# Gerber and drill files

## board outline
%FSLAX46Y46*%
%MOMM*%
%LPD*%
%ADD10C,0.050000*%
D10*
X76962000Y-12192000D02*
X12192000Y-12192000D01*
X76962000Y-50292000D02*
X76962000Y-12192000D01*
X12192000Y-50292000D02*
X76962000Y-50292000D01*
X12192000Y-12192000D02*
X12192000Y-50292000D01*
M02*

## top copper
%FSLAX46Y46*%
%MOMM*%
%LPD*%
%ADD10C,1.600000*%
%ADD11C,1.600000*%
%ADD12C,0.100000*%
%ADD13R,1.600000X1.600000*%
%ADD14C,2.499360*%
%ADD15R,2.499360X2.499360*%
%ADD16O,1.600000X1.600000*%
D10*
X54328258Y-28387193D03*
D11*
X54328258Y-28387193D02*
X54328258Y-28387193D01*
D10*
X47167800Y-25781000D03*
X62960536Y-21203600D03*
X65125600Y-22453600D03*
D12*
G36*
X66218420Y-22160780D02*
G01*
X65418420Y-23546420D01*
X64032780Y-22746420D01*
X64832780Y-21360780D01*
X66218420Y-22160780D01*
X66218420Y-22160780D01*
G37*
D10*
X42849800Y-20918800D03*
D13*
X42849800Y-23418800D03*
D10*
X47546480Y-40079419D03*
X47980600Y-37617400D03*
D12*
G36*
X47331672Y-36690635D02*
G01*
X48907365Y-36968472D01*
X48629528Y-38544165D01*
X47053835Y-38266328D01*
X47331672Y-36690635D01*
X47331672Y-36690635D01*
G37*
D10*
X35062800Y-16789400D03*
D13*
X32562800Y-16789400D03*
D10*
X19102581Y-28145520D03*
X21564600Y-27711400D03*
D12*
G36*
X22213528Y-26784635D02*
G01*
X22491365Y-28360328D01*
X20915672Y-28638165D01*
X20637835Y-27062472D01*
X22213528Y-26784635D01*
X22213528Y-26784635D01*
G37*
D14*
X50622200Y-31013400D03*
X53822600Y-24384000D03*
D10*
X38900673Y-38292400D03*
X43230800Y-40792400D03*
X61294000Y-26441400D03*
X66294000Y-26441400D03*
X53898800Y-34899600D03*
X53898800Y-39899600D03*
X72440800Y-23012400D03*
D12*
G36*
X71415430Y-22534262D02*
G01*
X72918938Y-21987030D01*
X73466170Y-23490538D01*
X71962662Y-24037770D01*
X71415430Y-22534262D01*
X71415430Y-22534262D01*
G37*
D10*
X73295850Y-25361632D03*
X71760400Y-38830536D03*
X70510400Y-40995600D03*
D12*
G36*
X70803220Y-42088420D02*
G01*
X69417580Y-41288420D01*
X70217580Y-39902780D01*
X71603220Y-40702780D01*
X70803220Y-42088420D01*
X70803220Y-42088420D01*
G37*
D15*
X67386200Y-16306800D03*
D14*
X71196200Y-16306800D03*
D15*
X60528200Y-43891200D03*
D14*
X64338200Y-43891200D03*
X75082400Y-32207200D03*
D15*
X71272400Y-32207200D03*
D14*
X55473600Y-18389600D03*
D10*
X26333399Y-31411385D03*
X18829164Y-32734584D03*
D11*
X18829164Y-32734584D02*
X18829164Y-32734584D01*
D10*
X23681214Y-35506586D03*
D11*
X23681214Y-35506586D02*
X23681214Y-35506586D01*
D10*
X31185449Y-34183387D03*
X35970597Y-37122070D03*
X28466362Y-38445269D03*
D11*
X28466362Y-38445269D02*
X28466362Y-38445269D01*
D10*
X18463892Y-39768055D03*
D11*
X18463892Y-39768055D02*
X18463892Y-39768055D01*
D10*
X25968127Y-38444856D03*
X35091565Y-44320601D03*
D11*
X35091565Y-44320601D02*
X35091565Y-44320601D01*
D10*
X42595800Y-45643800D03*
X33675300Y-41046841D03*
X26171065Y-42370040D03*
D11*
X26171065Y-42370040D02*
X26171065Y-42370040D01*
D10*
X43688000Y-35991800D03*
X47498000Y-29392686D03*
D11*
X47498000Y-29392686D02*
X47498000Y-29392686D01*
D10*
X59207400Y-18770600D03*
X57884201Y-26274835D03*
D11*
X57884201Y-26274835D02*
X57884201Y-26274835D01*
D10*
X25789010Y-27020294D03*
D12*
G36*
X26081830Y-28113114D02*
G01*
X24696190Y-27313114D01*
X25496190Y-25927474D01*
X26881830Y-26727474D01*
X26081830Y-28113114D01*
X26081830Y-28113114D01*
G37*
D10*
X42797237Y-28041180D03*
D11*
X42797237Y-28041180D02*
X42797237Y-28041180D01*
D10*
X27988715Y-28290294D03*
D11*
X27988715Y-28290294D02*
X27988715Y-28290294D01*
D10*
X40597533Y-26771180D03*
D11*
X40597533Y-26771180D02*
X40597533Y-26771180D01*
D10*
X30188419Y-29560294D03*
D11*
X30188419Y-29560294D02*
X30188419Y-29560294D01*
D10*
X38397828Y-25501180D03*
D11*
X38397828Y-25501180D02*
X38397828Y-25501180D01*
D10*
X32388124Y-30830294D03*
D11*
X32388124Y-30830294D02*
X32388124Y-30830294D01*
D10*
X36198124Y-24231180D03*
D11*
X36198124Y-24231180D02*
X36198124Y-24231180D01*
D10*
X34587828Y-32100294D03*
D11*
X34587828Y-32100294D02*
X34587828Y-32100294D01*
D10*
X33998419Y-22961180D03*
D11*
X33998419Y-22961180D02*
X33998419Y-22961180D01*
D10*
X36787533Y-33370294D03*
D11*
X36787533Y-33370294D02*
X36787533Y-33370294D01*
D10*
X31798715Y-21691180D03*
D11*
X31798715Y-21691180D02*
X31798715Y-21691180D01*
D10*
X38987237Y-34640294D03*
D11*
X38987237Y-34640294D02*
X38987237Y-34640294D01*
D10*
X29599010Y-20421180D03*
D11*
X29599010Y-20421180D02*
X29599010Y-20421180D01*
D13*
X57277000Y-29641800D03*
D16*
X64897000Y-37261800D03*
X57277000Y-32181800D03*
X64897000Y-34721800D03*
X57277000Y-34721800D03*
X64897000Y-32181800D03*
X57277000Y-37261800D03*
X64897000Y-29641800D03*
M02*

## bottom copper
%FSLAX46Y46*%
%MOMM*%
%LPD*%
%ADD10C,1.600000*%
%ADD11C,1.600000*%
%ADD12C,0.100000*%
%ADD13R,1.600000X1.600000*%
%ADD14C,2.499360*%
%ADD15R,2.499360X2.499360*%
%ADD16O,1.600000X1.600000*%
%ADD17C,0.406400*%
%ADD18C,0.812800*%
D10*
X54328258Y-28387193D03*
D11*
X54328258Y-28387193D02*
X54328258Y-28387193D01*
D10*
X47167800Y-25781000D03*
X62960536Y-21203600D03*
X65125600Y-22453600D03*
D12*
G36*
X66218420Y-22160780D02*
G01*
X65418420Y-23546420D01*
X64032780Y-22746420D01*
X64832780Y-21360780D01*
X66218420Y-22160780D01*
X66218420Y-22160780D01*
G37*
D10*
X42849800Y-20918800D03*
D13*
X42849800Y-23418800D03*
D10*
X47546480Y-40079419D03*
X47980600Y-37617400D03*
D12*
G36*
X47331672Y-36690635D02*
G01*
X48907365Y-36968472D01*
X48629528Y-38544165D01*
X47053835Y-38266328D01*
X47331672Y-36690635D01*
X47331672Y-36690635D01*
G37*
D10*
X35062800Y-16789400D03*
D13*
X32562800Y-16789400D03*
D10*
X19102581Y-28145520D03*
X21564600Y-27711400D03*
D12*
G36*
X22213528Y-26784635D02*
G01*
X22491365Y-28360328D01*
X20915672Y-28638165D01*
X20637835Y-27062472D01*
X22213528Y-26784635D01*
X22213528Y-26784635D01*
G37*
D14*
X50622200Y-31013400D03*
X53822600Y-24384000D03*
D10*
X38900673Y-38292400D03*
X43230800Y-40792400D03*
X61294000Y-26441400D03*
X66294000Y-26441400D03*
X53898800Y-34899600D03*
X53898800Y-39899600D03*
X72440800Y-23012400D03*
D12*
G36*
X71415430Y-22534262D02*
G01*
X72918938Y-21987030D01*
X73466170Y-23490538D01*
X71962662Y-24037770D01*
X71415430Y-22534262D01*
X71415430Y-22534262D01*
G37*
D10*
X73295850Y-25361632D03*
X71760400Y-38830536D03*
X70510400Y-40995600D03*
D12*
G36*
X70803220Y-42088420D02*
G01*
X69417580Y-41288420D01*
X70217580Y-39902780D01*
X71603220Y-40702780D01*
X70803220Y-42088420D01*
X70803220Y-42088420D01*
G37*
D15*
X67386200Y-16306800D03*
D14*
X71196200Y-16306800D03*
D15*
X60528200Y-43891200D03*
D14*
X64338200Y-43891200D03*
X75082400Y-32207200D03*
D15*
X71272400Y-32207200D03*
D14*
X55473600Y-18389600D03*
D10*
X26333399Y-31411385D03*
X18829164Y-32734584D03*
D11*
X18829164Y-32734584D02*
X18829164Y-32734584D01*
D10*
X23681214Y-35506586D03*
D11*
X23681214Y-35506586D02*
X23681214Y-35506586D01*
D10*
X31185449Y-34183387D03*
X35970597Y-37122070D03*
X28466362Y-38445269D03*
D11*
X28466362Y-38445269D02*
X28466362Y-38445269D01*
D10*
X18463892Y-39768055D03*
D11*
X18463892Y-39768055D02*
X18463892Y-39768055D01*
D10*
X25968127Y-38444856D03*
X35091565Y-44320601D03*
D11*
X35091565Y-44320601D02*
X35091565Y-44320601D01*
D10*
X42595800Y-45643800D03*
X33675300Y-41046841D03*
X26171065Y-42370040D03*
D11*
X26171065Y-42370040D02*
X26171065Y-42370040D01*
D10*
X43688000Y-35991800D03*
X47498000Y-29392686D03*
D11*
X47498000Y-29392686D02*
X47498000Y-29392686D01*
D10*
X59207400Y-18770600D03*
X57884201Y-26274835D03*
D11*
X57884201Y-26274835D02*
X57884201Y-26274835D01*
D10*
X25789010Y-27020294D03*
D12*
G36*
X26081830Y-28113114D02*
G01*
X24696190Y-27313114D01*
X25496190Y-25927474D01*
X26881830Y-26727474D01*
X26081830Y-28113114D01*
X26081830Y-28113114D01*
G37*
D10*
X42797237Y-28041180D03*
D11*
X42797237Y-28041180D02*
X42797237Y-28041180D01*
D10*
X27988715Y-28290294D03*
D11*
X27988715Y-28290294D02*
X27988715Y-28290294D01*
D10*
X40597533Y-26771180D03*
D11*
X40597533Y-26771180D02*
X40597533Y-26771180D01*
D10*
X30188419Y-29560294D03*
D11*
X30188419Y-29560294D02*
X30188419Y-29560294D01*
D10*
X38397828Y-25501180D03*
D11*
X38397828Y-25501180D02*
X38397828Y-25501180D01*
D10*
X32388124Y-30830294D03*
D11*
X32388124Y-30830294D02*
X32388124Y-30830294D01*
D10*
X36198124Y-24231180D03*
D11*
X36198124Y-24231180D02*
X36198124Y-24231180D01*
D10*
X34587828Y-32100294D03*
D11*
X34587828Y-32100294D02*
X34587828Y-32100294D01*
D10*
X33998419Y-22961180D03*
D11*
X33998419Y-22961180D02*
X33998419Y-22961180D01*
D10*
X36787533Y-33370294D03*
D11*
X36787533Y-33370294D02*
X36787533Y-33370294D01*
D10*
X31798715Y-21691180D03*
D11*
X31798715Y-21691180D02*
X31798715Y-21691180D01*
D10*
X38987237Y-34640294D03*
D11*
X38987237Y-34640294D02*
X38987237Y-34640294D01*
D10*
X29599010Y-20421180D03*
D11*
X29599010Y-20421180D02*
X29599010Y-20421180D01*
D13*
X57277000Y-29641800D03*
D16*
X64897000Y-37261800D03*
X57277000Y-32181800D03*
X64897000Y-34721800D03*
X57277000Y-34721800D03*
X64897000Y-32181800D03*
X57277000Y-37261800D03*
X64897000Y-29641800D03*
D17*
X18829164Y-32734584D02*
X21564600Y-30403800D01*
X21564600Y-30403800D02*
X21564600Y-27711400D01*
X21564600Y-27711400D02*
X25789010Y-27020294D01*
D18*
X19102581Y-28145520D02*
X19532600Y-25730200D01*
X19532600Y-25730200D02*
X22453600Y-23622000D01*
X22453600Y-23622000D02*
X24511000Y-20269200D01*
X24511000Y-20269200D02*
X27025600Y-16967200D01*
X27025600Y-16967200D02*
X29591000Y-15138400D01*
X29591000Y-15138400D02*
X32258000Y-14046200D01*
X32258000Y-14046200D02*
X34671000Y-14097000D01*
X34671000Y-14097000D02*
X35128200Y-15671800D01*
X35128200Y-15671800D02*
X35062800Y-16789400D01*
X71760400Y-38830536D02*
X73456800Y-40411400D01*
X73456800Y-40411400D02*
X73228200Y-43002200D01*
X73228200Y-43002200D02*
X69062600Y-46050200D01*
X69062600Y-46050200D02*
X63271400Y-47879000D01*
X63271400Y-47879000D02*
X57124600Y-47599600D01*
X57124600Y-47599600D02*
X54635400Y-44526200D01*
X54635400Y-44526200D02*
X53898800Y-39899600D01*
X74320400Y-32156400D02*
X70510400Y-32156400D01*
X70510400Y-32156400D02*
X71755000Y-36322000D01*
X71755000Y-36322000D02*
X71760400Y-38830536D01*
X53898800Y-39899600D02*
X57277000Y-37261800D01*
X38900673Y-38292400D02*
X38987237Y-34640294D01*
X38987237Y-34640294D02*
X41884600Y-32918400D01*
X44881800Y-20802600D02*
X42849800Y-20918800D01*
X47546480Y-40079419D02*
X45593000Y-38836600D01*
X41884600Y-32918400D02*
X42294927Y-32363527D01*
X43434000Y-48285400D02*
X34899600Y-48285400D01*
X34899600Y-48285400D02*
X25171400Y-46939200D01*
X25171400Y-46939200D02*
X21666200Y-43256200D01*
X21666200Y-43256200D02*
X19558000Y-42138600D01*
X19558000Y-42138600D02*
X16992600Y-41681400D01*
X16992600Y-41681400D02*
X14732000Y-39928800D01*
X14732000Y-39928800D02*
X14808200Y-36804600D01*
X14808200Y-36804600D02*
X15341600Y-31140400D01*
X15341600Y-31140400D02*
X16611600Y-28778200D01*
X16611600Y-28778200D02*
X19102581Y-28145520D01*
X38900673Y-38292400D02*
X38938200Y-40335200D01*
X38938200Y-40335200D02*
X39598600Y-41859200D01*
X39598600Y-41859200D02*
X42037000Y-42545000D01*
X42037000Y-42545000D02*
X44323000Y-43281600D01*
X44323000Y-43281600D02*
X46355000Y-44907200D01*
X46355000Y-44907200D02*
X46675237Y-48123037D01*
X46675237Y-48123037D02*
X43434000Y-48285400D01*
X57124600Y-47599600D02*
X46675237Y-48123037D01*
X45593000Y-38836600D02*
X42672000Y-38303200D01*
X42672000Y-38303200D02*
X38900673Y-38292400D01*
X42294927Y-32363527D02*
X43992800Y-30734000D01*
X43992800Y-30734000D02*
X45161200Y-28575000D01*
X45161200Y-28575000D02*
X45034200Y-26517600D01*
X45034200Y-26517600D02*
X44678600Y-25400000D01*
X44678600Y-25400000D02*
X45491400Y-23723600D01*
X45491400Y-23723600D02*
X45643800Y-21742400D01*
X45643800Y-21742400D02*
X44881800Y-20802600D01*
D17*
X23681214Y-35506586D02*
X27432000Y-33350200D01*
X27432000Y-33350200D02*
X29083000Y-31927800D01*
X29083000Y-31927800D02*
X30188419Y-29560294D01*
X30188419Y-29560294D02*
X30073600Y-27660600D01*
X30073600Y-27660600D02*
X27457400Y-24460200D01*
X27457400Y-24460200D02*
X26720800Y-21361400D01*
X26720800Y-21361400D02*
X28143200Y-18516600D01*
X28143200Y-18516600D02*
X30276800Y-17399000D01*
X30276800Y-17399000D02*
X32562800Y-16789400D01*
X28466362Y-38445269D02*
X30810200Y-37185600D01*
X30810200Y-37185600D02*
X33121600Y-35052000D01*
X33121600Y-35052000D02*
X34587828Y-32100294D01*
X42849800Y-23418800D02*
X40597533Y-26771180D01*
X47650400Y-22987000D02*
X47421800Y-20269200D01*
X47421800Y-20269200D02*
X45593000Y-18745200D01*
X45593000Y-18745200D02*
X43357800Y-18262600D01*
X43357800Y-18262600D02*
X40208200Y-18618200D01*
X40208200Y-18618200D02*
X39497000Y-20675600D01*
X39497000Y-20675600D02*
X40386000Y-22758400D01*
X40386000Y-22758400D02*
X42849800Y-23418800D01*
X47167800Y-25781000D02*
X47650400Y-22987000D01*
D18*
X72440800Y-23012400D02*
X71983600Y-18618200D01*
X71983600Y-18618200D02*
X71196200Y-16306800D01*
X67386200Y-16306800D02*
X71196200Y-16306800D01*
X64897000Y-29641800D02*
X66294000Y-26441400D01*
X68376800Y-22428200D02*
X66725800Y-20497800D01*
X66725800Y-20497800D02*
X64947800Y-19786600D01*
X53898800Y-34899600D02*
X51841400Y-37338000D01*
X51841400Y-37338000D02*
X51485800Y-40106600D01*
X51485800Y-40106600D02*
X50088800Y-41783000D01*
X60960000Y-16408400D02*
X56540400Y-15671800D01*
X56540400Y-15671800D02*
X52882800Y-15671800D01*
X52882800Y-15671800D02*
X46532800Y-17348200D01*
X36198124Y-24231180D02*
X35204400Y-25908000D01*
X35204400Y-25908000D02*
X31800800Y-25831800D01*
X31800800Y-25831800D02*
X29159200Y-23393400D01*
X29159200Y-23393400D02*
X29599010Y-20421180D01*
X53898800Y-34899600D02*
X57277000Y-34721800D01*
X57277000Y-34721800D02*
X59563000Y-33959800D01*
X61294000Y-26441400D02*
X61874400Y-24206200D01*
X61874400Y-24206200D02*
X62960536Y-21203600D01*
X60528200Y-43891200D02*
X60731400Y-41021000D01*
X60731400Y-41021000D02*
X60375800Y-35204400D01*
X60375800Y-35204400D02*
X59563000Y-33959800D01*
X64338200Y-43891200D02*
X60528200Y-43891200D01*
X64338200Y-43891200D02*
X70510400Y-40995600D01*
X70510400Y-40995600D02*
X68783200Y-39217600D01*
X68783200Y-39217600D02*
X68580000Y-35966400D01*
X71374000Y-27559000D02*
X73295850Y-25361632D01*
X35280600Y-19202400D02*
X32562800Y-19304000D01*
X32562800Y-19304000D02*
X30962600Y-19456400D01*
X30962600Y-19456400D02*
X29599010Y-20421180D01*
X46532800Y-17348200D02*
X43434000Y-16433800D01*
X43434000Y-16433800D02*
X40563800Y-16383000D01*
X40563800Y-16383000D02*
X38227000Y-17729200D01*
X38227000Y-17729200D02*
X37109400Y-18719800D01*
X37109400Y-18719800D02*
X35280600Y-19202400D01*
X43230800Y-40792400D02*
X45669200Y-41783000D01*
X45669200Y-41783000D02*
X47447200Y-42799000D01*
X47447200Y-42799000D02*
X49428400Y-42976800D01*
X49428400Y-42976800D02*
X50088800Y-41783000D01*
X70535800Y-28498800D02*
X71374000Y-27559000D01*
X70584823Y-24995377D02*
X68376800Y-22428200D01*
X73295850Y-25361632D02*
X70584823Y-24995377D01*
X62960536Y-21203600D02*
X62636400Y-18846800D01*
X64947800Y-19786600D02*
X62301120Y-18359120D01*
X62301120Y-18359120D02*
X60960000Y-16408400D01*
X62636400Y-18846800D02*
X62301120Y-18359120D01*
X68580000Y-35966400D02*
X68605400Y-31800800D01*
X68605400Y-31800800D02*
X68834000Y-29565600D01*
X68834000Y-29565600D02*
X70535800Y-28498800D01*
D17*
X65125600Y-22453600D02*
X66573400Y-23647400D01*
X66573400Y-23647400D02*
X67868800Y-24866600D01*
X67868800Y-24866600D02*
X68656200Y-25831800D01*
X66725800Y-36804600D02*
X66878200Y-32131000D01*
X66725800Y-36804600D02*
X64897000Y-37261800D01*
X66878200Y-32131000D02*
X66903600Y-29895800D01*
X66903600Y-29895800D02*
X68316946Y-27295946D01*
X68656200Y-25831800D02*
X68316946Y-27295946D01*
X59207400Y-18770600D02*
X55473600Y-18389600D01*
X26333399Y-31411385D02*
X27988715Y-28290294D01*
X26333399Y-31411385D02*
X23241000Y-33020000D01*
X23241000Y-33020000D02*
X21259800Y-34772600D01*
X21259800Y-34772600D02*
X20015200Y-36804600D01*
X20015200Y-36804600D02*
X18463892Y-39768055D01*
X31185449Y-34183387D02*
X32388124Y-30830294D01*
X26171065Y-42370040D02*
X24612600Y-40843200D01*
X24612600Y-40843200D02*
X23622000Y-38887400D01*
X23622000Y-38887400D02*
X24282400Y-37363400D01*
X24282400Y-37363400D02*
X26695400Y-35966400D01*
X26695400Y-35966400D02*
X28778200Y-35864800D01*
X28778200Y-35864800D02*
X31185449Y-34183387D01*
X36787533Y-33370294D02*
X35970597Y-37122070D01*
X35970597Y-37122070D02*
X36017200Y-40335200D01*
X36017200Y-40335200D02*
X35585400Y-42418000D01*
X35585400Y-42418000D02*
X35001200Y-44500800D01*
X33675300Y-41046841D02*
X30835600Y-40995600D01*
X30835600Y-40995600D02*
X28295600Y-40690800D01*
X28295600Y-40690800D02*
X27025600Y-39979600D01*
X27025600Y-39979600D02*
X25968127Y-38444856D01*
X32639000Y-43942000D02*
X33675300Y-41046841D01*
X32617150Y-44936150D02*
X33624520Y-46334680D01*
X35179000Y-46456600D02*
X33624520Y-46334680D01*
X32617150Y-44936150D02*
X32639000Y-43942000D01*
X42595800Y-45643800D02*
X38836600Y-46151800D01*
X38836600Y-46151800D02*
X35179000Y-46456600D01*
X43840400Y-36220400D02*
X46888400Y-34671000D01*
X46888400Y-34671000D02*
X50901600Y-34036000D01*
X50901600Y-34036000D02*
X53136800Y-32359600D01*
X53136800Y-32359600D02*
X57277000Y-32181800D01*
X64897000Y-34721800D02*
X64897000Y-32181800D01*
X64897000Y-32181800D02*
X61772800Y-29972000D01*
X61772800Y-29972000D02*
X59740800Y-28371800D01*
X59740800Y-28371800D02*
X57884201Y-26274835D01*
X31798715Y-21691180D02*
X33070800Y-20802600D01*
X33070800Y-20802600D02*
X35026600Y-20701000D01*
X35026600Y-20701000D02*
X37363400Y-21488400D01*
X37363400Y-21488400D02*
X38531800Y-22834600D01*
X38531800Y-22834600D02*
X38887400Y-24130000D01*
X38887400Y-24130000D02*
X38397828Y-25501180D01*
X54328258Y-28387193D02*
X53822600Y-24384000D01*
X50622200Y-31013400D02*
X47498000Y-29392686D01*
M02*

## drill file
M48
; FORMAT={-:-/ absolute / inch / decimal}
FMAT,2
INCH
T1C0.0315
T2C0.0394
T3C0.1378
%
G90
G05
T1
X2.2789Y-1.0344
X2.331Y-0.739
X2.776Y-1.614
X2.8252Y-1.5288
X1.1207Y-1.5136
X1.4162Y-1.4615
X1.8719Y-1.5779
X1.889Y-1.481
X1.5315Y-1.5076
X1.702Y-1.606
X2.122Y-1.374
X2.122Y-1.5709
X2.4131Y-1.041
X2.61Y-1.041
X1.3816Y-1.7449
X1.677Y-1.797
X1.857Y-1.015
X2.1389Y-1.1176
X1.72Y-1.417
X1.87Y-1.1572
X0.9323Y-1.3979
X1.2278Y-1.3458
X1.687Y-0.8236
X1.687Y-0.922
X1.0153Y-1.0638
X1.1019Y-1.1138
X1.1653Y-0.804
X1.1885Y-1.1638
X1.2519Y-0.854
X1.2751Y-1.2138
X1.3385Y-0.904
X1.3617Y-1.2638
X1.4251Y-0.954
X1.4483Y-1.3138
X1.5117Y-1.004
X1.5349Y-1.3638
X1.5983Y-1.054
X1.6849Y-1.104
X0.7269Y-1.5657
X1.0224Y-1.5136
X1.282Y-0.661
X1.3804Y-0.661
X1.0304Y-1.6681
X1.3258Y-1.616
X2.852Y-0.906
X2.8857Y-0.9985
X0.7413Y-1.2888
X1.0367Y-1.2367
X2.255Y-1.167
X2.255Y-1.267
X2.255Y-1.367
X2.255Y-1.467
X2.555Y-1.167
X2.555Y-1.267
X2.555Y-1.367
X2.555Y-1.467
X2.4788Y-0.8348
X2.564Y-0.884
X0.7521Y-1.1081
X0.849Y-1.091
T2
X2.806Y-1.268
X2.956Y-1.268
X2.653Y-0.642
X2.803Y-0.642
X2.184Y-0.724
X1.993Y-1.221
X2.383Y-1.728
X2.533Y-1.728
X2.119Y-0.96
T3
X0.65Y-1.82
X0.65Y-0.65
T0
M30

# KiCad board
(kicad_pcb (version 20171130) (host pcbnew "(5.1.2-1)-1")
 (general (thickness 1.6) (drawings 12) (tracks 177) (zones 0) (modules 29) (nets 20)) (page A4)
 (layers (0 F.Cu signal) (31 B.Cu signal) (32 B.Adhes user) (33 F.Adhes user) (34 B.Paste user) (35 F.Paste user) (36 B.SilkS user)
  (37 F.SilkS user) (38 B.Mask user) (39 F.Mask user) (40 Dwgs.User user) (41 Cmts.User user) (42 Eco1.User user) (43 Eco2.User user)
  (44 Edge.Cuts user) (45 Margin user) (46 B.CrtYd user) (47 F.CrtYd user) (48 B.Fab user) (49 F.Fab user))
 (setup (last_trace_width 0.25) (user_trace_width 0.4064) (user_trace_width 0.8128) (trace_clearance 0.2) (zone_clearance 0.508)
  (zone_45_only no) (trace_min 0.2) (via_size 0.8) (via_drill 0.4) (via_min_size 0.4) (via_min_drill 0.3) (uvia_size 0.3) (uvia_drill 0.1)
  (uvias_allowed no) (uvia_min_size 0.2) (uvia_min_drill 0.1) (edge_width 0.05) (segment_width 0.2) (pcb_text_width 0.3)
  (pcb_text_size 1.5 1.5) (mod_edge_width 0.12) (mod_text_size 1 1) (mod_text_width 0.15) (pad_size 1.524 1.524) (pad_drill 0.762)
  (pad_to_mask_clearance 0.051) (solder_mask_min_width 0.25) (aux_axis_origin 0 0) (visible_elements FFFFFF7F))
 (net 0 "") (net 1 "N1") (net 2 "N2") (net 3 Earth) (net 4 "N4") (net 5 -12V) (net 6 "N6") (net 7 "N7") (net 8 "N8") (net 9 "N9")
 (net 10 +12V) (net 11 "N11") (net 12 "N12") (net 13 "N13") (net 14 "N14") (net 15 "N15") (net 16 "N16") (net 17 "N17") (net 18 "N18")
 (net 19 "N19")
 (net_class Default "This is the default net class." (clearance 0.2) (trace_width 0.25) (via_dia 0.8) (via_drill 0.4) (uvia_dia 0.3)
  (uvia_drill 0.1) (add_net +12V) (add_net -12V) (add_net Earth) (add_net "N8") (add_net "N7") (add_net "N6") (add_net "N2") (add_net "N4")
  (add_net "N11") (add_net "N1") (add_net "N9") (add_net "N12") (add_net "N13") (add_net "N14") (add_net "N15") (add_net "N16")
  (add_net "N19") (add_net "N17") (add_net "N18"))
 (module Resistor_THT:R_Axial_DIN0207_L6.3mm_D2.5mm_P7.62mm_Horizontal (layer F.Cu) (at 47.1678 25.781 340)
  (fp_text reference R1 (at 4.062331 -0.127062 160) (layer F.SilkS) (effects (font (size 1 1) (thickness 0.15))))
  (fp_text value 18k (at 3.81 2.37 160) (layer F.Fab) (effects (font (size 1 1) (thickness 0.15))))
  (pad 2 thru_hole oval (at 7.62 0 340) (size 1.6 1.6) (drill 0.8) (layers *.Cu *.Mask) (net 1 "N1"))
  (pad 1 thru_hole circle (at 0 0 340) (size 1.6 1.6) (drill 0.8) (layers *.Cu *.Mask) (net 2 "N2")))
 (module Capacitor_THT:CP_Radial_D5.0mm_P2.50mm (layer F.Cu) (at 65.1256 22.4536 150)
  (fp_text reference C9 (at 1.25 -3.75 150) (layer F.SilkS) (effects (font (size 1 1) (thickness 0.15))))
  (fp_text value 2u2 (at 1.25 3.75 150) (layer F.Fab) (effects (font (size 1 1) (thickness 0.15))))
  (pad 2 thru_hole circle (at 2.5 0 150) (size 1.6 1.6) (drill 0.8) (layers *.Cu *.Mask) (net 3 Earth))
  (pad 1 thru_hole rect (at 0 0 150) (size 1.6 1.6) (drill 0.8) (layers *.Cu *.Mask) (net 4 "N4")))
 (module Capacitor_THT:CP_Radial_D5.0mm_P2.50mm (layer F.Cu) (at 42.8498 23.4188 90)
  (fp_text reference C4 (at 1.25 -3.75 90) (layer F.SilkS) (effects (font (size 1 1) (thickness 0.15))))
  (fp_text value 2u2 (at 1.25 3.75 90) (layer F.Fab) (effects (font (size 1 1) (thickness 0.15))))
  (pad 2 thru_hole circle (at 2.5 0 90) (size 1.6 1.6) (drill 0.8) (layers *.Cu *.Mask) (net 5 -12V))
  (pad 1 thru_hole rect (at 0 0 90) (size 1.6 1.6) (drill 0.8) (layers *.Cu *.Mask) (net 2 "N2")))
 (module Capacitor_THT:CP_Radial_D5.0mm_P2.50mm (layer F.Cu) (at 47.9806 37.6174 260)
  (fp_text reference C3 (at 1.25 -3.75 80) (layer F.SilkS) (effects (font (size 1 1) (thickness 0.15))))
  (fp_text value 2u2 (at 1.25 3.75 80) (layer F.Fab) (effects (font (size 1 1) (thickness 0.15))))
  (pad 2 thru_hole circle (at 2.5 0 260) (size 1.6 1.6) (drill 0.8) (layers *.Cu *.Mask) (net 5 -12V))
  (pad 1 thru_hole rect (at 0 0 260) (size 1.6 1.6) (drill 0.8) (layers *.Cu *.Mask) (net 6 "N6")))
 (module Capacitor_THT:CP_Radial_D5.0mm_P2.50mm (layer F.Cu) (at 32.5628 16.7894)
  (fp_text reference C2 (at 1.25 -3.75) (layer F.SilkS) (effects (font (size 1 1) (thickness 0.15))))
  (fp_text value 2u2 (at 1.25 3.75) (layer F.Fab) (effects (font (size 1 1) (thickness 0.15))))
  (pad 2 thru_hole circle (at 2.5 0) (size 1.6 1.6) (drill 0.8) (layers *.Cu *.Mask) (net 5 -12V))
  (pad 1 thru_hole rect (at 0 0) (size 1.6 1.6) (drill 0.8) (layers *.Cu *.Mask) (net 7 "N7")))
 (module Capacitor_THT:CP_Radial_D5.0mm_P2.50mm (layer F.Cu) (at 21.5646 27.7114 190)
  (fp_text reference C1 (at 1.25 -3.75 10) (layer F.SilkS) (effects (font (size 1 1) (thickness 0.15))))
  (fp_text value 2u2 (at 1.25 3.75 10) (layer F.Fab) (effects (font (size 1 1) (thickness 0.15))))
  (pad 2 thru_hole circle (at 2.5 0 190) (size 1.6 1.6) (drill 0.8) (layers *.Cu *.Mask) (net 5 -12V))
  (pad 1 thru_hole rect (at 0 0 190) (size 1.6 1.6) (drill 0.8) (layers *.Cu *.Mask) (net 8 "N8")))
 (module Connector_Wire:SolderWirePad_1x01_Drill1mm (layer F.Cu) (at 50.6222 31.0134 340)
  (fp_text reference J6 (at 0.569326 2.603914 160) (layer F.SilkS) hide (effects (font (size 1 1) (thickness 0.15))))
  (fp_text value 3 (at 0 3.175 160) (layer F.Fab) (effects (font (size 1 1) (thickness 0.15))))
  (pad 1 thru_hole circle (at 0 0 340) (size 2.49936 2.49936) (drill 1.00076) (layers *.Cu *.Mask) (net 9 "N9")))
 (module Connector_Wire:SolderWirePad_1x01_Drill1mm (layer F.Cu) (at 53.8226 24.384 340)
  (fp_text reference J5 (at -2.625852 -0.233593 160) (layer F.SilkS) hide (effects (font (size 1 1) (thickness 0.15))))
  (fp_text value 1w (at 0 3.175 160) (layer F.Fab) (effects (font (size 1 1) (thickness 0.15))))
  (pad 1 thru_hole circle (at 0 0 340) (size 2.49936 2.49936) (drill 1.00076) (layers *.Cu *.Mask) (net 1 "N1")))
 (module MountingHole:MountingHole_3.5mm (layer F.Cu) (at 16.51 46.228)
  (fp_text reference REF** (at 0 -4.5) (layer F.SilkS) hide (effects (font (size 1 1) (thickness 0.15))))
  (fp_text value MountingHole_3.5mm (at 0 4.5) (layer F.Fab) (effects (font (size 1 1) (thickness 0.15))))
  (pad 1 np_thru_hole circle (at 0 0) (size 3.5 3.5) (drill 3.5) (layers *.Cu *.Mask)))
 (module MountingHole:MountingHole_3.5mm (layer F.Cu) (at 16.51 16.51)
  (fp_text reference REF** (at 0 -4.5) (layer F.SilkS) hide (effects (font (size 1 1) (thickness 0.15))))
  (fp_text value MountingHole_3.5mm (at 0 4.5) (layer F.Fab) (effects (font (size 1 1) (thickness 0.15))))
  (pad 1 np_thru_hole circle (at 0 0) (size 3.5 3.5) (drill 3.5) (layers *.Cu *.Mask)))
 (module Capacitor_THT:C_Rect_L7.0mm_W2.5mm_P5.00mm (layer F.Cu) (at 43.2308 40.7924 150)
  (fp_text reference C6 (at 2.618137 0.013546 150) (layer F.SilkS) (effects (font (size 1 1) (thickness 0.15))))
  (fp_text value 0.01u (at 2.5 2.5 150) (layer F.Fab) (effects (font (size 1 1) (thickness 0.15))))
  (pad 2 thru_hole circle (at 5 0 150) (size 1.6 1.6) (drill 0.8) (layers *.Cu *.Mask) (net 5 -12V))
  (pad 1 thru_hole circle (at 0 0 150) (size 1.6 1.6) (drill 0.8) (layers *.Cu *.Mask) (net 3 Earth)))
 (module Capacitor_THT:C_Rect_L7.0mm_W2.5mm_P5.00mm (layer F.Cu) (at 66.294 26.4414 180)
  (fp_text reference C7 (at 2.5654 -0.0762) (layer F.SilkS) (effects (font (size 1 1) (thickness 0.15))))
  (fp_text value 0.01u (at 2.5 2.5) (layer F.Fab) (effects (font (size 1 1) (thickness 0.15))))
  (pad 2 thru_hole circle (at 5 0 180) (size 1.6 1.6) (drill 0.8) (layers *.Cu *.Mask) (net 3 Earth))
  (pad 1 thru_hole circle (at 0 0 180) (size 1.6 1.6) (drill 0.8) (layers *.Cu *.Mask) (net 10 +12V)))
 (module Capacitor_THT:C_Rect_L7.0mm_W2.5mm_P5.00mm (layer F.Cu) (at 53.8988 34.8996 270)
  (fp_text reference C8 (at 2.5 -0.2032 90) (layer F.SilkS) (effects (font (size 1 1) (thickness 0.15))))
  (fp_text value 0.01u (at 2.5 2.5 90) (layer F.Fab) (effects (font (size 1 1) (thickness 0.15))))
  (pad 1 thru_hole circle (at 0 0 270) (size 1.6 1.6) (drill 0.8) (layers *.Cu *.Mask) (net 3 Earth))
  (pad 2 thru_hole circle (at 5 0 270) (size 1.6 1.6) (drill 0.8) (layers *.Cu *.Mask) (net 5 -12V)))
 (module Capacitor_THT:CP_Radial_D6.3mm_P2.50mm (layer F.Cu) (at 72.4408 23.0124 290)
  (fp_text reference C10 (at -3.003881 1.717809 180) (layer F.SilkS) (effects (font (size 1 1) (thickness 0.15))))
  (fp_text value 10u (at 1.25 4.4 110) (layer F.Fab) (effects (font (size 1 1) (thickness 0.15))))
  (pad 1 thru_hole rect (at 0 0 290) (size 1.6 1.6) (drill 0.8) (layers *.Cu *.Mask) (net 10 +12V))
  (pad 2 thru_hole circle (at 2.5 0 290) (size 1.6 1.6) (drill 0.8) (layers *.Cu *.Mask) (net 3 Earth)))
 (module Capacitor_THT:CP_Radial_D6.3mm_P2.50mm (layer F.Cu) (at 70.5104 40.9956 60)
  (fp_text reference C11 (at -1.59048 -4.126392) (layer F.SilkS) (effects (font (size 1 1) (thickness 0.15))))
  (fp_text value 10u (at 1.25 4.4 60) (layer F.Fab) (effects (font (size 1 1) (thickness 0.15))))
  (pad 2 thru_hole circle (at 2.5 0 60) (size 1.6 1.6) (drill 0.8) (layers *.Cu *.Mask) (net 5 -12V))
  (pad 1 thru_hole rect (at 0 0 60) (size 1.6 1.6) (drill 0.8) (layers *.Cu *.Mask) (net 3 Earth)))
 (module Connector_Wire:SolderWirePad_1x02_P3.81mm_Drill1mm (layer F.Cu) (at 67.3862 16.3068)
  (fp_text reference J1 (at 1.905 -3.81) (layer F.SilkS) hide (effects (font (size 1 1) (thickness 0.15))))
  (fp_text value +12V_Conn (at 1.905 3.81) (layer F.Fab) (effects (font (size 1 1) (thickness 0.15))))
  (pad 1 thru_hole rect (at 0 0) (size 2.49936 2.49936) (drill 1.00076) (layers *.Cu *.Mask) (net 10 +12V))
  (pad 2 thru_hole circle (at 3.81 0) (size 2.49936 2.49936) (drill 1.00076) (layers *.Cu *.Mask) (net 10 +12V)))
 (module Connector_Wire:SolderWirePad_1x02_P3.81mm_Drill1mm (layer F.Cu) (at 60.5282 43.8912)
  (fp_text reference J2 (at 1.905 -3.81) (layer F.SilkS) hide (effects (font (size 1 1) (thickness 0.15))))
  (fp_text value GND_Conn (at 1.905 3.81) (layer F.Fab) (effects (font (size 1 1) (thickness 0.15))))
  (pad 1 thru_hole rect (at 0 0) (size 2.49936 2.49936) (drill 1.00076) (layers *.Cu *.Mask) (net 3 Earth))
  (pad 2 thru_hole circle (at 3.81 0) (size 2.49936 2.49936) (drill 1.00076) (layers *.Cu *.Mask) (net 3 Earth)))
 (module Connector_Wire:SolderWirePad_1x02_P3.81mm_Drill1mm (layer F.Cu) (at 71.2724 32.2072)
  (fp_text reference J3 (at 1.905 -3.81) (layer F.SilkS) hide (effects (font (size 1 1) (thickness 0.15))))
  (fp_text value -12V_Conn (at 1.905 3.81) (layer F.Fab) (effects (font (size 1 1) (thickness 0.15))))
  (pad 2 thru_hole circle (at 3.81 0) (size 2.49936 2.49936) (drill 1.00076) (layers *.Cu *.Mask) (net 5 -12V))
  (pad 1 thru_hole rect (at 0 0) (size 2.49936 2.49936) (drill 1.00076) (layers *.Cu *.Mask) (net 5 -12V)))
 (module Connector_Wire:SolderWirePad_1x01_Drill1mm (layer F.Cu) (at 55.4736 18.3896 350)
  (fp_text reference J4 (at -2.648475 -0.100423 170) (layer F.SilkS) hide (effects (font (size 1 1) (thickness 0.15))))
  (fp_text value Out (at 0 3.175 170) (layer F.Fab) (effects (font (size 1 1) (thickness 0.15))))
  (pad 1 thru_hole circle (at 0 0 350) (size 2.49936 2.49936) (drill 1.00076) (layers *.Cu *.Mask) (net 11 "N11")))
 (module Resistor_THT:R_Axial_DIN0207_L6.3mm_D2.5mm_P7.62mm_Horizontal (layer F.Cu) (at 26.333399 31.411385 190)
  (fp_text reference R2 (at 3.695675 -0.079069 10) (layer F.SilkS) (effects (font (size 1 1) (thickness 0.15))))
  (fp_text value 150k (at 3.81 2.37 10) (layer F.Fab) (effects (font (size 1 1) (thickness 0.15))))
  (pad 1 thru_hole circle (at 0 0 190) (size 1.6 1.6) (drill 0.8) (layers *.Cu *.Mask) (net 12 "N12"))
  (pad 2 thru_hole oval (at 7.62 0 190) (size 1.6 1.6) (drill 0.8) (layers *.Cu *.Mask) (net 8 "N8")))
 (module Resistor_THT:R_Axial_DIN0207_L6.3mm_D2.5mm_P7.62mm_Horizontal (layer F.Cu) (at 31.185449 34.183387 190)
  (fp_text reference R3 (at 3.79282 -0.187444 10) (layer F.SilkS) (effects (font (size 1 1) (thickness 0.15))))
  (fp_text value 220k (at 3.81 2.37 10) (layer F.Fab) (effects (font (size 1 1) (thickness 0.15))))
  (pad 2 thru_hole oval (at 7.62 0 190) (size 1.6 1.6) (drill 0.8) (layers *.Cu *.Mask) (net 7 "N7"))
  (pad 1 thru_hole circle (at 0 0 190) (size 1.6 1.6) (drill 0.8) (layers *.Cu *.Mask) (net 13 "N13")))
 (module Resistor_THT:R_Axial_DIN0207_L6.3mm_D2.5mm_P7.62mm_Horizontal (layer F.Cu) (at 35.970597 37.12207 190)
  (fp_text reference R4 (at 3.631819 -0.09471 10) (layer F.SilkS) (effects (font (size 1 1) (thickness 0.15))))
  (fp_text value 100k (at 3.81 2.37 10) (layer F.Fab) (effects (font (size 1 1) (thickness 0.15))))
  (pad 1 thru_hole circle (at 0 0 190) (size 1.6 1.6) (drill 0.8) (layers *.Cu *.Mask) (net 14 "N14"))
  (pad 2 thru_hole oval (at 7.62 0 190) (size 1.6 1.6) (drill 0.8) (layers *.Cu *.Mask) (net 6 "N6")))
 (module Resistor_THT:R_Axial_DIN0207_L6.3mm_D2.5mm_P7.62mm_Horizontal (layer F.Cu) (at 25.968127 38.444856 190)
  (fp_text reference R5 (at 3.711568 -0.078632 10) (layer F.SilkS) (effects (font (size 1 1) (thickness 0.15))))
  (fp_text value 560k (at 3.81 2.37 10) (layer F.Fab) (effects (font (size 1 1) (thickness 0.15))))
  (pad 2 thru_hole oval (at 7.62 0 190) (size 1.6 1.6) (drill 0.8) (layers *.Cu *.Mask) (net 12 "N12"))
  (pad 1 thru_hole circle (at 0 0 190) (size 1.6 1.6) (drill 0.8) (layers *.Cu *.Mask) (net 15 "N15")))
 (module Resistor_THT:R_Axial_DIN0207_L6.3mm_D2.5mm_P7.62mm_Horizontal (layer F.Cu) (at 42.5958 45.6438 170)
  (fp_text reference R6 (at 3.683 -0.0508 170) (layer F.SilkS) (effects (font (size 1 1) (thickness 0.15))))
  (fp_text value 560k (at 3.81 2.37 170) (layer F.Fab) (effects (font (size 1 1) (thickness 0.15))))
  (pad 2 thru_hole oval (at 7.62 0 170) (size 1.6 1.6) (drill 0.8) (layers *.Cu *.Mask) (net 14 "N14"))
  (pad 1 thru_hole circle (at 0 0 170) (size 1.6 1.6) (drill 0.8) (layers *.Cu *.Mask) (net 15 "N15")))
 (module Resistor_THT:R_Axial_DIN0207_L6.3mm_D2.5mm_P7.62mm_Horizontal (layer F.Cu) (at 33.6753 41.046841 190)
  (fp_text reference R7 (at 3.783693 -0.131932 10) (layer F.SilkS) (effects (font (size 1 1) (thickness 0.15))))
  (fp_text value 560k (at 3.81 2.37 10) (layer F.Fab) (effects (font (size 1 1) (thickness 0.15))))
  (pad 1 thru_hole circle (at 0 0 190) (size 1.6 1.6) (drill 0.8) (layers *.Cu *.Mask) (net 15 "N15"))
  (pad 2 thru_hole oval (at 7.62 0 190) (size 1.6 1.6) (drill 0.8) (layers *.Cu *.Mask) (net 13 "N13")))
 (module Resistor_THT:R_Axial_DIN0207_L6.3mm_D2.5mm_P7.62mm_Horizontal (layer F.Cu) (at 43.688 35.9918 60)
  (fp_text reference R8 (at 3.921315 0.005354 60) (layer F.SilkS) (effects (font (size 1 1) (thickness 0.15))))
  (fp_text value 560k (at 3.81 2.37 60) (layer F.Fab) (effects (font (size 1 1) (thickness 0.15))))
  (pad 1 thru_hole circle (at 0 0 60) (size 1.6 1.6) (drill 0.8) (layers *.Cu *.Mask) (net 15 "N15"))
  (pad 2 thru_hole oval (at 7.62 0 60) (size 1.6 1.6) (drill 0.8) (layers *.Cu *.Mask) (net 9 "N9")))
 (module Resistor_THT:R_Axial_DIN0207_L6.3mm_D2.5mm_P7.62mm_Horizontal (layer F.Cu) (at 59.2074 18.7706 260)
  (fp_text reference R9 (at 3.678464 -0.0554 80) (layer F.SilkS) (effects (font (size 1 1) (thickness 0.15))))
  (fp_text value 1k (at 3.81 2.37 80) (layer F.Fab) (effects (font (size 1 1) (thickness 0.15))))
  (pad 1 thru_hole circle (at 0 0 260) (size 1.6 1.6) (drill 0.8) (layers *.Cu *.Mask) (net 11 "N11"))
  (pad 2 thru_hole oval (at 7.62 0 260) (size 1.6 1.6) (drill 0.8) (layers *.Cu *.Mask) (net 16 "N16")))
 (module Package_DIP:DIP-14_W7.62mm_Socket (layer F.Cu) (at 25.78901 27.020294 60)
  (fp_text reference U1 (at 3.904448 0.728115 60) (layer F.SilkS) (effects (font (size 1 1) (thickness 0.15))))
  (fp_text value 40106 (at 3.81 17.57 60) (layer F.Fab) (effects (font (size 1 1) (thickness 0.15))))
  (pad 1 thru_hole rect (at 0 0 60) (size 1.6 1.6) (drill 0.8) (layers *.Cu *.Mask) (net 8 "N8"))
  (pad 8 thru_hole oval (at 7.62 15.24 60) (size 1.6 1.6) (drill 0.8) (layers *.Cu *.Mask) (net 9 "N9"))
  (pad 2 thru_hole oval (at 0 2.54 60) (size 1.6 1.6) (drill 0.8) (layers *.Cu *.Mask) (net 12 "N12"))
  (pad 9 thru_hole oval (at 7.62 12.7 60) (size 1.6 1.6) (drill 0.8) (layers *.Cu *.Mask) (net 2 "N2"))
  (pad 3 thru_hole oval (at 0 5.08 60) (size 1.6 1.6) (drill 0.8) (layers *.Cu *.Mask) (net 7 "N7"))
  (pad 10 thru_hole oval (at 7.62 10.16 60) (size 1.6 1.6) (drill 0.8) (layers *.Cu *.Mask) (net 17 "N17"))
  (pad 4 thru_hole oval (at 0 7.62 60) (size 1.6 1.6) (drill 0.8) (layers *.Cu *.Mask) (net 13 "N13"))
  (pad 11 thru_hole oval (at 7.62 7.62 60) (size 1.6 1.6) (drill 0.8) (layers *.Cu *.Mask) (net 3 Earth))
  (pad 5 thru_hole oval (at 0 10.16 60) (size 1.6 1.6) (drill 0.8) (layers *.Cu *.Mask) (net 6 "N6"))
  (pad 12 thru_hole oval (at 7.62 5.08 60) (size 1.6 1.6) (drill 0.8) (layers *.Cu *.Mask) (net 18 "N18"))
  (pad 6 thru_hole oval (at 0 12.7 60) (size 1.6 1.6) (drill 0.8) (layers *.Cu *.Mask) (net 14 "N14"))
  (pad 13 thru_hole oval (at 7.62 2.54 60) (size 1.6 1.6) (drill 0.8) (layers *.Cu *.Mask) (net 17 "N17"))
  (pad 7 thru_hole oval (at 0 15.24 60) (size 1.6 1.6) (drill 0.8) (layers *.Cu *.Mask) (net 5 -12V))
  (pad 14 thru_hole oval (at 7.62 0 60) (size 1.6 1.6) (drill 0.8) (layers *.Cu *.Mask) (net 3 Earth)))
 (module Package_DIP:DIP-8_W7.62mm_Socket (layer F.Cu) (at 57.277 29.6418)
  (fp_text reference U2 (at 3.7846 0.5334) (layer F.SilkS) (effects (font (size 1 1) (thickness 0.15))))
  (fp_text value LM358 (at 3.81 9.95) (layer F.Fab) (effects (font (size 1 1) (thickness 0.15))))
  (pad 1 thru_hole rect (at 0 0) (size 1.6 1.6) (drill 0.8) (layers *.Cu *.Mask) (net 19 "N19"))
  (pad 5 thru_hole oval (at 7.62 7.62) (size 1.6 1.6) (drill 0.8) (layers *.Cu *.Mask) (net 4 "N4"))
  (pad 2 thru_hole oval (at 0 2.54) (size 1.6 1.6) (drill 0.8) (layers *.Cu *.Mask) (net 15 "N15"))
  (pad 6 thru_hole oval (at 7.62 5.08) (size 1.6 1.6) (drill 0.8) (layers *.Cu *.Mask) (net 16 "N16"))
  (pad 3 thru_hole oval (at 0 5.08) (size 1.6 1.6) (drill 0.8) (layers *.Cu *.Mask) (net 3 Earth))
  (pad 7 thru_hole oval (at 7.62 2.54) (size 1.6 1.6) (drill 0.8) (layers *.Cu *.Mask) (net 16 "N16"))
  (pad 4 thru_hole oval (at 0 7.62) (size 1.6 1.6) (drill 0.8) (layers *.Cu *.Mask) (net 5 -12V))
  (pad 8 thru_hole oval (at 7.62 0) (size 1.6 1.6) (drill 0.8) (layers *.Cu *.Mask) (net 10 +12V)))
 (gr_line (start 76.962 12.192) (end 12.192 12.192) (layer Edge.Cuts) (width 0.05))
 (gr_line (start 76.962 50.292) (end 76.962 12.192) (layer Edge.Cuts) (width 0.05))
 (gr_line (start 12.192 50.292) (end 76.962 50.292) (layer Edge.Cuts) (width 0.05))
 (gr_line (start 12.192 12.192) (end 12.192 50.292) (layer Edge.Cuts) (width 0.05))
 (segment (start 18.829164 32.734584) (end 21.5646 30.4038) (width 0.4064) (layer B.Cu) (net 8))
 (segment (start 21.5646 30.4038) (end 21.5646 27.7114) (width 0.4064) (layer B.Cu) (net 8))
 (segment (start 21.5646 27.7114) (end 25.78901 27.020294) (width 0.4064) (layer B.Cu) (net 8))
 (segment (start 19.102581 28.14552) (end 19.5326 25.7302) (width 0.8128) (layer B.Cu) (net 5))
 (segment (start 19.5326 25.7302) (end 22.4536 23.622) (width 0.8128) (layer B.Cu) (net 5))
 (segment (start 22.4536 23.622) (end 24.511 20.2692) (width 0.8128) (layer B.Cu) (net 5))
 (segment (start 24.511 20.2692) (end 27.0256 16.9672) (width 0.8128) (layer B.Cu) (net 5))
 (segment (start 27.0256 16.9672) (end 29.591 15.1384) (width 0.8128) (layer B.Cu) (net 5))
 (segment (start 29.591 15.1384) (end 32.258 14.0462) (width 0.8128) (layer B.Cu) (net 5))
 (segment (start 32.258 14.0462) (end 34.671 14.097) (width 0.8128) (layer B.Cu) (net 5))
 (segment (start 34.671 14.097) (end 35.1282 15.6718) (width 0.8128) (layer B.Cu) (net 5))
 (segment (start 35.1282 15.6718) (end 35.0628 16.7894) (width 0.8128) (layer B.Cu) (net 5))
 (segment (start 71.7604 38.830536) (end 73.4568 40.4114) (width 0.8128) (layer B.Cu) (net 5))
 (segment (start 73.4568 40.4114) (end 73.2282 43.0022) (width 0.8128) (layer B.Cu) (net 5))
 (segment (start 73.2282 43.0022) (end 69.0626 46.0502) (width 0.8128) (layer B.Cu) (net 5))
 (segment (start 69.0626 46.0502) (end 63.2714 47.879) (width 0.8128) (layer B.Cu) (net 5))
 (segment (start 63.2714 47.879) (end 57.1246 47.5996) (width 0.8128) (layer B.Cu) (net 5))
 (segment (start 57.1246 47.5996) (end 54.6354 44.5262) (width 0.8128) (layer B.Cu) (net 5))
 (segment (start 54.6354 44.5262) (end 53.8988 39.8996) (width 0.8128) (layer B.Cu) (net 5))
 (segment (start 74.3204 32.1564) (end 70.5104 32.1564) (width 0.8128) (layer B.Cu) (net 5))
 (segment (start 70.5104 32.1564) (end 71.755 36.322) (width 0.8128) (layer B.Cu) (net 5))
 (segment (start 71.755 36.322) (end 71.7604 38.830536) (width 0.8128) (layer B.Cu) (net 5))
 (segment (start 53.8988 39.8996) (end 57.277 37.2618) (width 0.8128) (layer B.Cu) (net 5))
 (segment (start 38.900673 38.2924) (end 38.987237 34.640294) (width 0.8128) (layer B.Cu) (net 5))
 (segment (start 38.987237 34.640294) (end 41.8846 32.9184) (width 0.8128) (layer B.Cu) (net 5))
 (segment (start 44.8818 20.8026) (end 42.8498 20.9188) (width 0.8128) (layer B.Cu) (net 5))
 (segment (start 47.54648 40.079419) (end 45.593 38.8366) (width 0.8128) (layer B.Cu) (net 5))
 (segment (start 41.8846 32.9184) (end 42.294927 32.363527) (width 0.8128) (layer B.Cu) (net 5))
 (segment (start 43.434 48.2854) (end 34.8996 48.2854) (width 0.8128) (layer B.Cu) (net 5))
 (segment (start 34.8996 48.2854) (end 25.1714 46.9392) (width 0.8128) (layer B.Cu) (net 5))
 (segment (start 25.1714 46.9392) (end 21.6662 43.2562) (width 0.8128) (layer B.Cu) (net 5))
 (segment (start 21.6662 43.2562) (end 19.558 42.1386) (width 0.8128) (layer B.Cu) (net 5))
 (segment (start 19.558 42.1386) (end 16.9926 41.6814) (width 0.8128) (layer B.Cu) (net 5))
 (segment (start 16.9926 41.6814) (end 14.732 39.9288) (width 0.8128) (layer B.Cu) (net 5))
 (segment (start 14.732 39.9288) (end 14.8082 36.8046) (width 0.8128) (layer B.Cu) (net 5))
 (segment (start 14.8082 36.8046) (end 15.3416 31.1404) (width 0.8128) (layer B.Cu) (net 5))
 (segment (start 15.3416 31.1404) (end 16.6116 28.7782) (width 0.8128) (layer B.Cu) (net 5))
 (segment (start 16.6116 28.7782) (end 19.102581 28.14552) (width 0.8128) (layer B.Cu) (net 5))
 (segment (start 38.900673 38.2924) (end 38.9382 40.3352) (width 0.8128) (layer B.Cu) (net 5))
 (segment (start 38.9382 40.3352) (end 39.5986 41.8592) (width 0.8128) (layer B.Cu) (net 5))
 (segment (start 39.5986 41.8592) (end 42.037 42.545) (width 0.8128) (layer B.Cu) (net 5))
 (segment (start 42.037 42.545) (end 44.323 43.2816) (width 0.8128) (layer B.Cu) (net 5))
 (segment (start 44.323 43.2816) (end 46.355 44.9072) (width 0.8128) (layer B.Cu) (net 5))
 (segment (start 46.355 44.9072) (end 46.675237 48.123037) (width 0.8128) (layer B.Cu) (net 5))
 (segment (start 46.675237 48.123037) (end 43.434 48.2854) (width 0.8128) (layer B.Cu) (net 5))
 (segment (start 57.1246 47.5996) (end 46.675237 48.123037) (width 0.8128) (layer B.Cu) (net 5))
 (segment (start 45.593 38.8366) (end 42.672 38.3032) (width 0.8128) (layer B.Cu) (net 5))
 (segment (start 42.672 38.3032) (end 38.900673 38.2924) (width 0.8128) (layer B.Cu) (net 5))
 (segment (start 42.294927 32.363527) (end 43.9928 30.734) (width 0.8128) (layer B.Cu) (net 5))
 (segment (start 43.9928 30.734) (end 45.1612 28.575) (width 0.8128) (layer B.Cu) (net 5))
 (segment (start 45.1612 28.575) (end 45.0342 26.5176) (width 0.8128) (layer B.Cu) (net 5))
 (segment (start 45.0342 26.5176) (end 44.6786 25.4) (width 0.8128) (layer B.Cu) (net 5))
 (segment (start 44.6786 25.4) (end 45.4914 23.7236) (width 0.8128) (layer B.Cu) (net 5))
 (segment (start 45.4914 23.7236) (end 45.6438 21.7424) (width 0.8128) (layer B.Cu) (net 5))
 (segment (start 45.6438 21.7424) (end 44.8818 20.8026) (width 0.8128) (layer B.Cu) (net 5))
 (segment (start 23.681214 35.506586) (end 27.432 33.3502) (width 0.4064) (layer B.Cu) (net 7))
 (segment (start 27.432 33.3502) (end 29.083 31.9278) (width 0.4064) (layer B.Cu) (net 7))
 (segment (start 29.083 31.9278) (end 30.188419 29.560294) (width 0.4064) (layer B.Cu) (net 7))
 (segment (start 30.188419 29.560294) (end 30.0736 27.6606) (width 0.4064) (layer B.Cu) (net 7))
 (segment (start 30.0736 27.6606) (end 27.4574 24.4602) (width 0.4064) (layer B.Cu) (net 7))
 (segment (start 27.4574 24.4602) (end 26.7208 21.3614) (width 0.4064) (layer B.Cu) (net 7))
 (segment (start 26.7208 21.3614) (end 28.1432 18.5166) (width 0.4064) (layer B.Cu) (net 7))
 (segment (start 28.1432 18.5166) (end 30.2768 17.399) (width 0.4064) (layer B.Cu) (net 7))
 (segment (start 30.2768 17.399) (end 32.5628 16.7894) (width 0.4064) (layer B.Cu) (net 7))
 (segment (start 28.466362 38.445269) (end 30.8102 37.1856) (width 0.4064) (layer B.Cu) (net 6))
 (segment (start 30.8102 37.1856) (end 33.1216 35.052) (width 0.4064) (layer B.Cu) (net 6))
 (segment (start 33.1216 35.052) (end 34.587828 32.100294) (width 0.4064) (layer B.Cu) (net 6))
 (segment (start 42.8498 23.4188) (end 40.597533 26.77118) (width 0.4064) (layer B.Cu) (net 2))
 (segment (start 47.6504 22.987) (end 47.4218 20.2692) (width 0.4064) (layer B.Cu) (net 2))
 (segment (start 47.4218 20.2692) (end 45.593 18.7452) (width 0.4064) (layer B.Cu) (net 2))
 (segment (start 45.593 18.7452) (end 43.3578 18.2626) (width 0.4064) (layer B.Cu) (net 2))
 (segment (start 43.3578 18.2626) (end 40.2082 18.6182) (width 0.4064) (layer B.Cu) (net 2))
 (segment (start 40.2082 18.6182) (end 39.497 20.6756) (width 0.4064) (layer B.Cu) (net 2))
 (segment (start 39.497 20.6756) (end 40.386 22.7584) (width 0.4064) (layer B.Cu) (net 2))
 (segment (start 40.386 22.7584) (end 42.8498 23.4188) (width 0.4064) (layer B.Cu) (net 2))
 (segment (start 47.1678 25.781) (end 47.6504 22.987) (width 0.4064) (layer B.Cu) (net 2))
 (segment (start 72.4408 23.0124) (end 71.9836 18.6182) (width 0.8128) (layer B.Cu) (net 10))
 (segment (start 71.9836 18.6182) (end 71.1962 16.3068) (width 0.8128) (layer B.Cu) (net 10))
 (segment (start 67.3862 16.3068) (end 71.1962 16.3068) (width 0.8128) (layer B.Cu) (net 10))
 (segment (start 64.897 29.6418) (end 66.294 26.4414) (width 0.8128) (layer B.Cu) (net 10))
 (segment (start 68.3768 22.4282) (end 66.7258 20.4978) (width 0.8128) (layer B.Cu) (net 3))
 (segment (start 66.7258 20.4978) (end 64.9478 19.7866) (width 0.8128) (layer B.Cu) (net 3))
 (segment (start 53.8988 34.8996) (end 51.8414 37.338) (width 0.8128) (layer B.Cu) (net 3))
 (segment (start 51.8414 37.338) (end 51.4858 40.1066) (width 0.8128) (layer B.Cu) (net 3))
 (segment (start 51.4858 40.1066) (end 50.0888 41.783) (width 0.8128) (layer B.Cu) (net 3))
 (segment (start 60.96 16.4084) (end 56.5404 15.6718) (width 0.8128) (layer B.Cu) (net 3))
 (segment (start 56.5404 15.6718) (end 52.8828 15.6718) (width 0.8128) (layer B.Cu) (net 3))
 (segment (start 52.8828 15.6718) (end 46.5328 17.3482) (width 0.8128) (layer B.Cu) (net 3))
 (segment (start 36.198124 24.23118) (end 35.2044 25.908) (width 0.8128) (layer B.Cu) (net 3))
 (segment (start 35.2044 25.908) (end 31.8008 25.8318) (width 0.8128) (layer B.Cu) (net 3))
 (segment (start 31.8008 25.8318) (end 29.1592 23.3934) (width 0.8128) (layer B.Cu) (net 3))
 (segment (start 29.1592 23.3934) (end 29.59901 20.42118) (width 0.8128) (layer B.Cu) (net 3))
 (segment (start 53.8988 34.8996) (end 57.277 34.7218) (width 0.8128) (layer B.Cu) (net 3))
 (segment (start 57.277 34.7218) (end 59.563 33.9598) (width 0.8128) (layer B.Cu) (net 3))
 (segment (start 61.294 26.4414) (end 61.8744 24.2062) (width 0.8128) (layer B.Cu) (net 3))
 (segment (start 61.8744 24.2062) (end 62.960536 21.2036) (width 0.8128) (layer B.Cu) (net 3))
 (segment (start 60.5282 43.8912) (end 60.7314 41.021) (width 0.8128) (layer B.Cu) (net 3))
 (segment (start 60.7314 41.021) (end 60.3758 35.2044) (width 0.8128) (layer B.Cu) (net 3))
 (segment (start 60.3758 35.2044) (end 59.563 33.9598) (width 0.8128) (layer B.Cu) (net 3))
 (segment (start 64.3382 43.8912) (end 60.5282 43.8912) (width 0.8128) (layer B.Cu) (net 3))
 (segment (start 64.3382 43.8912) (end 70.5104 40.9956) (width 0.8128) (layer B.Cu) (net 3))
 (segment (start 70.5104 40.9956) (end 68.7832 39.2176) (width 0.8128) (layer B.Cu) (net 3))
 (segment (start 68.7832 39.2176) (end 68.58 35.9664) (width 0.8128) (layer B.Cu) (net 3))
 (segment (start 71.374 27.559) (end 73.29585 25.361632) (width 0.8128) (layer B.Cu) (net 3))
 (segment (start 35.2806 19.2024) (end 32.5628 19.304) (width 0.8128) (layer B.Cu) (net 3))
 (segment (start 32.5628 19.304) (end 30.9626 19.4564) (width 0.8128) (layer B.Cu) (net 3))
 (segment (start 30.9626 19.4564) (end 29.59901 20.42118) (width 0.8128) (layer B.Cu) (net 3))
 (segment (start 46.5328 17.3482) (end 43.434 16.4338) (width 0.8128) (layer B.Cu) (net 3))
 (segment (start 43.434 16.4338) (end 40.5638 16.383) (width 0.8128) (layer B.Cu) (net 3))
 (segment (start 40.5638 16.383) (end 38.227 17.7292) (width 0.8128) (layer B.Cu) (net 3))
 (segment (start 38.227 17.7292) (end 37.1094 18.7198) (width 0.8128) (layer B.Cu) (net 3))
 (segment (start 37.1094 18.7198) (end 35.2806 19.2024) (width 0.8128) (layer B.Cu) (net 3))
 (segment (start 43.2308 40.7924) (end 45.6692 41.783) (width 0.8128) (layer B.Cu) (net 3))
 (segment (start 45.6692 41.783) (end 47.4472 42.799) (width 0.8128) (layer B.Cu) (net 3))
 (segment (start 47.4472 42.799) (end 49.4284 42.9768) (width 0.8128) (layer B.Cu) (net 3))
 (segment (start 49.4284 42.9768) (end 50.0888 41.783) (width 0.8128) (layer B.Cu) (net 3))
 (segment (start 70.5358 28.4988) (end 71.374 27.559) (width 0.8128) (layer B.Cu) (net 3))
 (segment (start 70.584823 24.995377) (end 68.3768 22.4282) (width 0.8128) (layer B.Cu) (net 3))
 (segment (start 73.29585 25.361632) (end 70.584823 24.995377) (width 0.8128) (layer B.Cu) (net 3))
 (segment (start 62.960536 21.2036) (end 62.6364 18.8468) (width 0.8128) (layer B.Cu) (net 3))
 (segment (start 64.9478 19.7866) (end 62.30112 18.35912) (width 0.8128) (layer B.Cu) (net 3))
 (segment (start 62.30112 18.35912) (end 60.96 16.4084) (width 0.8128) (layer B.Cu) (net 3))
 (segment (start 62.6364 18.8468) (end 62.30112 18.35912) (width 0.8128) (layer B.Cu) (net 3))
 (segment (start 68.58 35.9664) (end 68.6054 31.8008) (width 0.8128) (layer B.Cu) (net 3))
 (segment (start 68.6054 31.8008) (end 68.834 29.5656) (width 0.8128) (layer B.Cu) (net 3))
 (segment (start 68.834 29.5656) (end 70.5358 28.4988) (width 0.8128) (layer B.Cu) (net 3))
 (segment (start 65.1256 22.4536) (end 66.5734 23.6474) (width 0.4064) (layer B.Cu) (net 4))
 (segment (start 66.5734 23.6474) (end 67.8688 24.8666) (width 0.4064) (layer B.Cu) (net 4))
 (segment (start 67.8688 24.8666) (end 68.6562 25.8318) (width 0.4064) (layer B.Cu) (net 4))
 (segment (start 66.7258 36.8046) (end 66.8782 32.131) (width 0.4064) (layer B.Cu) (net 4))
 (segment (start 66.7258 36.8046) (end 64.897 37.2618) (width 0.4064) (layer B.Cu) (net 4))
 (segment (start 66.8782 32.131) (end 66.9036 29.8958) (width 0.4064) (layer B.Cu) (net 4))
 (segment (start 66.9036 29.8958) (end 68.316946 27.295946) (width 0.4064) (layer B.Cu) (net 4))
 (segment (start 68.6562 25.8318) (end 68.316946 27.295946) (width 0.4064) (layer B.Cu) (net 4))
 (segment (start 59.2074 18.7706) (end 55.4736 18.3896) (width 0.4064) (layer B.Cu) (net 11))
 (segment (start 26.333399 31.411385) (end 27.988715 28.290294) (width 0.4064) (layer B.Cu) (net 12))
 (segment (start 26.333399 31.411385) (end 23.241 33.02) (width 0.4064) (layer B.Cu) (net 12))
 (segment (start 23.241 33.02) (end 21.2598 34.7726) (width 0.4064) (layer B.Cu) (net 12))
 (segment (start 21.2598 34.7726) (end 20.0152 36.8046) (width 0.4064) (layer B.Cu) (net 12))
 (segment (start 20.0152 36.8046) (end 18.463892 39.768055) (width 0.4064) (layer B.Cu) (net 12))
 (segment (start 31.185449 34.183387) (end 32.388124 30.830294) (width 0.4064) (layer B.Cu) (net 13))
 (segment (start 26.171065 42.37004) (end 24.6126 40.8432) (width 0.4064) (layer B.Cu) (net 13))
 (segment (start 24.6126 40.8432) (end 23.622 38.8874) (width 0.4064) (layer B.Cu) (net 13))
 (segment (start 23.622 38.8874) (end 24.2824 37.3634) (width 0.4064) (layer B.Cu) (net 13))
 (segment (start 24.2824 37.3634) (end 26.6954 35.9664) (width 0.4064) (layer B.Cu) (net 13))
 (segment (start 26.6954 35.9664) (end 28.7782 35.8648) (width 0.4064) (layer B.Cu) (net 13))
 (segment (start 28.7782 35.8648) (end 31.185449 34.183387) (width 0.4064) (layer B.Cu) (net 13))
 (segment (start 36.787533 33.370294) (end 35.970597 37.12207) (width 0.4064) (layer B.Cu) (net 14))
 (segment (start 35.970597 37.12207) (end 36.0172 40.3352) (width 0.4064) (layer B.Cu) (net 14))
 (segment (start 36.0172 40.3352) (end 35.5854 42.418) (width 0.4064) (layer B.Cu) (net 14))
 (segment (start 35.5854 42.418) (end 35.0012 44.5008) (width 0.4064) (layer B.Cu) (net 14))
 (segment (start 33.6753 41.046841) (end 30.8356 40.9956) (width 0.4064) (layer B.Cu) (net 15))
 (segment (start 30.8356 40.9956) (end 28.2956 40.6908) (width 0.4064) (layer B.Cu) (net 15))
 (segment (start 28.2956 40.6908) (end 27.0256 39.9796) (width 0.4064) (layer B.Cu) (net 15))
 (segment (start 27.0256 39.9796) (end 25.968127 38.444856) (width 0.4064) (layer B.Cu) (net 15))
 (segment (start 32.639 43.942) (end 33.6753 41.046841) (width 0.4064) (layer B.Cu) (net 15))
 (segment (start 32.61715 44.93615) (end 33.62452 46.33468) (width 0.4064) (layer B.Cu) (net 15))
 (segment (start 35.179 46.4566) (end 33.62452 46.33468) (width 0.4064) (layer B.Cu) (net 15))
 (segment (start 32.61715 44.93615) (end 32.639 43.942) (width 0.4064) (layer B.Cu) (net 15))
 (segment (start 42.5958 45.6438) (end 38.8366 46.1518) (width 0.4064) (layer B.Cu) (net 15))
 (segment (start 38.8366 46.1518) (end 35.179 46.4566) (width 0.4064) (layer B.Cu) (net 15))
 (segment (start 43.8404 36.2204) (end 46.8884 34.671) (width 0.4064) (layer B.Cu) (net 15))
 (segment (start 46.8884 34.671) (end 50.9016 34.036) (width 0.4064) (layer B.Cu) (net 15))
 (segment (start 50.9016 34.036) (end 53.1368 32.3596) (width 0.4064) (layer B.Cu) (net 15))
 (segment (start 53.1368 32.3596) (end 57.277 32.1818) (width 0.4064) (layer B.Cu) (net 15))
 (segment (start 64.897 34.7218) (end 64.897 32.1818) (width 0.4064) (layer B.Cu) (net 16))
 (segment (start 64.897 32.1818) (end 61.7728 29.972) (width 0.4064) (layer B.Cu) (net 16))
 (segment (start 61.7728 29.972) (end 59.7408 28.3718) (width 0.4064) (layer B.Cu) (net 16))
 (segment (start 59.7408 28.3718) (end 57.884201 26.274835) (width 0.4064) (layer B.Cu) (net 16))
 (segment (start 31.798715 21.69118) (end 33.0708 20.8026) (width 0.4064) (layer B.Cu) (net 17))
 (segment (start 33.0708 20.8026) (end 35.0266 20.701) (width 0.4064) (layer B.Cu) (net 17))
 (segment (start 35.0266 20.701) (end 37.3634 21.4884) (width 0.4064) (layer B.Cu) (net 17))
 (segment (start 37.3634 21.4884) (end 38.5318 22.8346) (width 0.4064) (layer B.Cu) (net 17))
 (segment (start 38.5318 22.8346) (end 38.8874 24.13) (width 0.4064) (layer B.Cu) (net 17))
 (segment (start 38.8874 24.13) (end 38.397828 25.50118) (width 0.4064) (layer B.Cu) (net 17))
 (segment (start 54.328258 28.387193) (end 53.8226 24.384) (width 0.4064) (layer B.Cu) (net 1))
 (segment (start 50.6222 31.0134) (end 47.498 29.392686) (width 0.4064) (layer B.Cu) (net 9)))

